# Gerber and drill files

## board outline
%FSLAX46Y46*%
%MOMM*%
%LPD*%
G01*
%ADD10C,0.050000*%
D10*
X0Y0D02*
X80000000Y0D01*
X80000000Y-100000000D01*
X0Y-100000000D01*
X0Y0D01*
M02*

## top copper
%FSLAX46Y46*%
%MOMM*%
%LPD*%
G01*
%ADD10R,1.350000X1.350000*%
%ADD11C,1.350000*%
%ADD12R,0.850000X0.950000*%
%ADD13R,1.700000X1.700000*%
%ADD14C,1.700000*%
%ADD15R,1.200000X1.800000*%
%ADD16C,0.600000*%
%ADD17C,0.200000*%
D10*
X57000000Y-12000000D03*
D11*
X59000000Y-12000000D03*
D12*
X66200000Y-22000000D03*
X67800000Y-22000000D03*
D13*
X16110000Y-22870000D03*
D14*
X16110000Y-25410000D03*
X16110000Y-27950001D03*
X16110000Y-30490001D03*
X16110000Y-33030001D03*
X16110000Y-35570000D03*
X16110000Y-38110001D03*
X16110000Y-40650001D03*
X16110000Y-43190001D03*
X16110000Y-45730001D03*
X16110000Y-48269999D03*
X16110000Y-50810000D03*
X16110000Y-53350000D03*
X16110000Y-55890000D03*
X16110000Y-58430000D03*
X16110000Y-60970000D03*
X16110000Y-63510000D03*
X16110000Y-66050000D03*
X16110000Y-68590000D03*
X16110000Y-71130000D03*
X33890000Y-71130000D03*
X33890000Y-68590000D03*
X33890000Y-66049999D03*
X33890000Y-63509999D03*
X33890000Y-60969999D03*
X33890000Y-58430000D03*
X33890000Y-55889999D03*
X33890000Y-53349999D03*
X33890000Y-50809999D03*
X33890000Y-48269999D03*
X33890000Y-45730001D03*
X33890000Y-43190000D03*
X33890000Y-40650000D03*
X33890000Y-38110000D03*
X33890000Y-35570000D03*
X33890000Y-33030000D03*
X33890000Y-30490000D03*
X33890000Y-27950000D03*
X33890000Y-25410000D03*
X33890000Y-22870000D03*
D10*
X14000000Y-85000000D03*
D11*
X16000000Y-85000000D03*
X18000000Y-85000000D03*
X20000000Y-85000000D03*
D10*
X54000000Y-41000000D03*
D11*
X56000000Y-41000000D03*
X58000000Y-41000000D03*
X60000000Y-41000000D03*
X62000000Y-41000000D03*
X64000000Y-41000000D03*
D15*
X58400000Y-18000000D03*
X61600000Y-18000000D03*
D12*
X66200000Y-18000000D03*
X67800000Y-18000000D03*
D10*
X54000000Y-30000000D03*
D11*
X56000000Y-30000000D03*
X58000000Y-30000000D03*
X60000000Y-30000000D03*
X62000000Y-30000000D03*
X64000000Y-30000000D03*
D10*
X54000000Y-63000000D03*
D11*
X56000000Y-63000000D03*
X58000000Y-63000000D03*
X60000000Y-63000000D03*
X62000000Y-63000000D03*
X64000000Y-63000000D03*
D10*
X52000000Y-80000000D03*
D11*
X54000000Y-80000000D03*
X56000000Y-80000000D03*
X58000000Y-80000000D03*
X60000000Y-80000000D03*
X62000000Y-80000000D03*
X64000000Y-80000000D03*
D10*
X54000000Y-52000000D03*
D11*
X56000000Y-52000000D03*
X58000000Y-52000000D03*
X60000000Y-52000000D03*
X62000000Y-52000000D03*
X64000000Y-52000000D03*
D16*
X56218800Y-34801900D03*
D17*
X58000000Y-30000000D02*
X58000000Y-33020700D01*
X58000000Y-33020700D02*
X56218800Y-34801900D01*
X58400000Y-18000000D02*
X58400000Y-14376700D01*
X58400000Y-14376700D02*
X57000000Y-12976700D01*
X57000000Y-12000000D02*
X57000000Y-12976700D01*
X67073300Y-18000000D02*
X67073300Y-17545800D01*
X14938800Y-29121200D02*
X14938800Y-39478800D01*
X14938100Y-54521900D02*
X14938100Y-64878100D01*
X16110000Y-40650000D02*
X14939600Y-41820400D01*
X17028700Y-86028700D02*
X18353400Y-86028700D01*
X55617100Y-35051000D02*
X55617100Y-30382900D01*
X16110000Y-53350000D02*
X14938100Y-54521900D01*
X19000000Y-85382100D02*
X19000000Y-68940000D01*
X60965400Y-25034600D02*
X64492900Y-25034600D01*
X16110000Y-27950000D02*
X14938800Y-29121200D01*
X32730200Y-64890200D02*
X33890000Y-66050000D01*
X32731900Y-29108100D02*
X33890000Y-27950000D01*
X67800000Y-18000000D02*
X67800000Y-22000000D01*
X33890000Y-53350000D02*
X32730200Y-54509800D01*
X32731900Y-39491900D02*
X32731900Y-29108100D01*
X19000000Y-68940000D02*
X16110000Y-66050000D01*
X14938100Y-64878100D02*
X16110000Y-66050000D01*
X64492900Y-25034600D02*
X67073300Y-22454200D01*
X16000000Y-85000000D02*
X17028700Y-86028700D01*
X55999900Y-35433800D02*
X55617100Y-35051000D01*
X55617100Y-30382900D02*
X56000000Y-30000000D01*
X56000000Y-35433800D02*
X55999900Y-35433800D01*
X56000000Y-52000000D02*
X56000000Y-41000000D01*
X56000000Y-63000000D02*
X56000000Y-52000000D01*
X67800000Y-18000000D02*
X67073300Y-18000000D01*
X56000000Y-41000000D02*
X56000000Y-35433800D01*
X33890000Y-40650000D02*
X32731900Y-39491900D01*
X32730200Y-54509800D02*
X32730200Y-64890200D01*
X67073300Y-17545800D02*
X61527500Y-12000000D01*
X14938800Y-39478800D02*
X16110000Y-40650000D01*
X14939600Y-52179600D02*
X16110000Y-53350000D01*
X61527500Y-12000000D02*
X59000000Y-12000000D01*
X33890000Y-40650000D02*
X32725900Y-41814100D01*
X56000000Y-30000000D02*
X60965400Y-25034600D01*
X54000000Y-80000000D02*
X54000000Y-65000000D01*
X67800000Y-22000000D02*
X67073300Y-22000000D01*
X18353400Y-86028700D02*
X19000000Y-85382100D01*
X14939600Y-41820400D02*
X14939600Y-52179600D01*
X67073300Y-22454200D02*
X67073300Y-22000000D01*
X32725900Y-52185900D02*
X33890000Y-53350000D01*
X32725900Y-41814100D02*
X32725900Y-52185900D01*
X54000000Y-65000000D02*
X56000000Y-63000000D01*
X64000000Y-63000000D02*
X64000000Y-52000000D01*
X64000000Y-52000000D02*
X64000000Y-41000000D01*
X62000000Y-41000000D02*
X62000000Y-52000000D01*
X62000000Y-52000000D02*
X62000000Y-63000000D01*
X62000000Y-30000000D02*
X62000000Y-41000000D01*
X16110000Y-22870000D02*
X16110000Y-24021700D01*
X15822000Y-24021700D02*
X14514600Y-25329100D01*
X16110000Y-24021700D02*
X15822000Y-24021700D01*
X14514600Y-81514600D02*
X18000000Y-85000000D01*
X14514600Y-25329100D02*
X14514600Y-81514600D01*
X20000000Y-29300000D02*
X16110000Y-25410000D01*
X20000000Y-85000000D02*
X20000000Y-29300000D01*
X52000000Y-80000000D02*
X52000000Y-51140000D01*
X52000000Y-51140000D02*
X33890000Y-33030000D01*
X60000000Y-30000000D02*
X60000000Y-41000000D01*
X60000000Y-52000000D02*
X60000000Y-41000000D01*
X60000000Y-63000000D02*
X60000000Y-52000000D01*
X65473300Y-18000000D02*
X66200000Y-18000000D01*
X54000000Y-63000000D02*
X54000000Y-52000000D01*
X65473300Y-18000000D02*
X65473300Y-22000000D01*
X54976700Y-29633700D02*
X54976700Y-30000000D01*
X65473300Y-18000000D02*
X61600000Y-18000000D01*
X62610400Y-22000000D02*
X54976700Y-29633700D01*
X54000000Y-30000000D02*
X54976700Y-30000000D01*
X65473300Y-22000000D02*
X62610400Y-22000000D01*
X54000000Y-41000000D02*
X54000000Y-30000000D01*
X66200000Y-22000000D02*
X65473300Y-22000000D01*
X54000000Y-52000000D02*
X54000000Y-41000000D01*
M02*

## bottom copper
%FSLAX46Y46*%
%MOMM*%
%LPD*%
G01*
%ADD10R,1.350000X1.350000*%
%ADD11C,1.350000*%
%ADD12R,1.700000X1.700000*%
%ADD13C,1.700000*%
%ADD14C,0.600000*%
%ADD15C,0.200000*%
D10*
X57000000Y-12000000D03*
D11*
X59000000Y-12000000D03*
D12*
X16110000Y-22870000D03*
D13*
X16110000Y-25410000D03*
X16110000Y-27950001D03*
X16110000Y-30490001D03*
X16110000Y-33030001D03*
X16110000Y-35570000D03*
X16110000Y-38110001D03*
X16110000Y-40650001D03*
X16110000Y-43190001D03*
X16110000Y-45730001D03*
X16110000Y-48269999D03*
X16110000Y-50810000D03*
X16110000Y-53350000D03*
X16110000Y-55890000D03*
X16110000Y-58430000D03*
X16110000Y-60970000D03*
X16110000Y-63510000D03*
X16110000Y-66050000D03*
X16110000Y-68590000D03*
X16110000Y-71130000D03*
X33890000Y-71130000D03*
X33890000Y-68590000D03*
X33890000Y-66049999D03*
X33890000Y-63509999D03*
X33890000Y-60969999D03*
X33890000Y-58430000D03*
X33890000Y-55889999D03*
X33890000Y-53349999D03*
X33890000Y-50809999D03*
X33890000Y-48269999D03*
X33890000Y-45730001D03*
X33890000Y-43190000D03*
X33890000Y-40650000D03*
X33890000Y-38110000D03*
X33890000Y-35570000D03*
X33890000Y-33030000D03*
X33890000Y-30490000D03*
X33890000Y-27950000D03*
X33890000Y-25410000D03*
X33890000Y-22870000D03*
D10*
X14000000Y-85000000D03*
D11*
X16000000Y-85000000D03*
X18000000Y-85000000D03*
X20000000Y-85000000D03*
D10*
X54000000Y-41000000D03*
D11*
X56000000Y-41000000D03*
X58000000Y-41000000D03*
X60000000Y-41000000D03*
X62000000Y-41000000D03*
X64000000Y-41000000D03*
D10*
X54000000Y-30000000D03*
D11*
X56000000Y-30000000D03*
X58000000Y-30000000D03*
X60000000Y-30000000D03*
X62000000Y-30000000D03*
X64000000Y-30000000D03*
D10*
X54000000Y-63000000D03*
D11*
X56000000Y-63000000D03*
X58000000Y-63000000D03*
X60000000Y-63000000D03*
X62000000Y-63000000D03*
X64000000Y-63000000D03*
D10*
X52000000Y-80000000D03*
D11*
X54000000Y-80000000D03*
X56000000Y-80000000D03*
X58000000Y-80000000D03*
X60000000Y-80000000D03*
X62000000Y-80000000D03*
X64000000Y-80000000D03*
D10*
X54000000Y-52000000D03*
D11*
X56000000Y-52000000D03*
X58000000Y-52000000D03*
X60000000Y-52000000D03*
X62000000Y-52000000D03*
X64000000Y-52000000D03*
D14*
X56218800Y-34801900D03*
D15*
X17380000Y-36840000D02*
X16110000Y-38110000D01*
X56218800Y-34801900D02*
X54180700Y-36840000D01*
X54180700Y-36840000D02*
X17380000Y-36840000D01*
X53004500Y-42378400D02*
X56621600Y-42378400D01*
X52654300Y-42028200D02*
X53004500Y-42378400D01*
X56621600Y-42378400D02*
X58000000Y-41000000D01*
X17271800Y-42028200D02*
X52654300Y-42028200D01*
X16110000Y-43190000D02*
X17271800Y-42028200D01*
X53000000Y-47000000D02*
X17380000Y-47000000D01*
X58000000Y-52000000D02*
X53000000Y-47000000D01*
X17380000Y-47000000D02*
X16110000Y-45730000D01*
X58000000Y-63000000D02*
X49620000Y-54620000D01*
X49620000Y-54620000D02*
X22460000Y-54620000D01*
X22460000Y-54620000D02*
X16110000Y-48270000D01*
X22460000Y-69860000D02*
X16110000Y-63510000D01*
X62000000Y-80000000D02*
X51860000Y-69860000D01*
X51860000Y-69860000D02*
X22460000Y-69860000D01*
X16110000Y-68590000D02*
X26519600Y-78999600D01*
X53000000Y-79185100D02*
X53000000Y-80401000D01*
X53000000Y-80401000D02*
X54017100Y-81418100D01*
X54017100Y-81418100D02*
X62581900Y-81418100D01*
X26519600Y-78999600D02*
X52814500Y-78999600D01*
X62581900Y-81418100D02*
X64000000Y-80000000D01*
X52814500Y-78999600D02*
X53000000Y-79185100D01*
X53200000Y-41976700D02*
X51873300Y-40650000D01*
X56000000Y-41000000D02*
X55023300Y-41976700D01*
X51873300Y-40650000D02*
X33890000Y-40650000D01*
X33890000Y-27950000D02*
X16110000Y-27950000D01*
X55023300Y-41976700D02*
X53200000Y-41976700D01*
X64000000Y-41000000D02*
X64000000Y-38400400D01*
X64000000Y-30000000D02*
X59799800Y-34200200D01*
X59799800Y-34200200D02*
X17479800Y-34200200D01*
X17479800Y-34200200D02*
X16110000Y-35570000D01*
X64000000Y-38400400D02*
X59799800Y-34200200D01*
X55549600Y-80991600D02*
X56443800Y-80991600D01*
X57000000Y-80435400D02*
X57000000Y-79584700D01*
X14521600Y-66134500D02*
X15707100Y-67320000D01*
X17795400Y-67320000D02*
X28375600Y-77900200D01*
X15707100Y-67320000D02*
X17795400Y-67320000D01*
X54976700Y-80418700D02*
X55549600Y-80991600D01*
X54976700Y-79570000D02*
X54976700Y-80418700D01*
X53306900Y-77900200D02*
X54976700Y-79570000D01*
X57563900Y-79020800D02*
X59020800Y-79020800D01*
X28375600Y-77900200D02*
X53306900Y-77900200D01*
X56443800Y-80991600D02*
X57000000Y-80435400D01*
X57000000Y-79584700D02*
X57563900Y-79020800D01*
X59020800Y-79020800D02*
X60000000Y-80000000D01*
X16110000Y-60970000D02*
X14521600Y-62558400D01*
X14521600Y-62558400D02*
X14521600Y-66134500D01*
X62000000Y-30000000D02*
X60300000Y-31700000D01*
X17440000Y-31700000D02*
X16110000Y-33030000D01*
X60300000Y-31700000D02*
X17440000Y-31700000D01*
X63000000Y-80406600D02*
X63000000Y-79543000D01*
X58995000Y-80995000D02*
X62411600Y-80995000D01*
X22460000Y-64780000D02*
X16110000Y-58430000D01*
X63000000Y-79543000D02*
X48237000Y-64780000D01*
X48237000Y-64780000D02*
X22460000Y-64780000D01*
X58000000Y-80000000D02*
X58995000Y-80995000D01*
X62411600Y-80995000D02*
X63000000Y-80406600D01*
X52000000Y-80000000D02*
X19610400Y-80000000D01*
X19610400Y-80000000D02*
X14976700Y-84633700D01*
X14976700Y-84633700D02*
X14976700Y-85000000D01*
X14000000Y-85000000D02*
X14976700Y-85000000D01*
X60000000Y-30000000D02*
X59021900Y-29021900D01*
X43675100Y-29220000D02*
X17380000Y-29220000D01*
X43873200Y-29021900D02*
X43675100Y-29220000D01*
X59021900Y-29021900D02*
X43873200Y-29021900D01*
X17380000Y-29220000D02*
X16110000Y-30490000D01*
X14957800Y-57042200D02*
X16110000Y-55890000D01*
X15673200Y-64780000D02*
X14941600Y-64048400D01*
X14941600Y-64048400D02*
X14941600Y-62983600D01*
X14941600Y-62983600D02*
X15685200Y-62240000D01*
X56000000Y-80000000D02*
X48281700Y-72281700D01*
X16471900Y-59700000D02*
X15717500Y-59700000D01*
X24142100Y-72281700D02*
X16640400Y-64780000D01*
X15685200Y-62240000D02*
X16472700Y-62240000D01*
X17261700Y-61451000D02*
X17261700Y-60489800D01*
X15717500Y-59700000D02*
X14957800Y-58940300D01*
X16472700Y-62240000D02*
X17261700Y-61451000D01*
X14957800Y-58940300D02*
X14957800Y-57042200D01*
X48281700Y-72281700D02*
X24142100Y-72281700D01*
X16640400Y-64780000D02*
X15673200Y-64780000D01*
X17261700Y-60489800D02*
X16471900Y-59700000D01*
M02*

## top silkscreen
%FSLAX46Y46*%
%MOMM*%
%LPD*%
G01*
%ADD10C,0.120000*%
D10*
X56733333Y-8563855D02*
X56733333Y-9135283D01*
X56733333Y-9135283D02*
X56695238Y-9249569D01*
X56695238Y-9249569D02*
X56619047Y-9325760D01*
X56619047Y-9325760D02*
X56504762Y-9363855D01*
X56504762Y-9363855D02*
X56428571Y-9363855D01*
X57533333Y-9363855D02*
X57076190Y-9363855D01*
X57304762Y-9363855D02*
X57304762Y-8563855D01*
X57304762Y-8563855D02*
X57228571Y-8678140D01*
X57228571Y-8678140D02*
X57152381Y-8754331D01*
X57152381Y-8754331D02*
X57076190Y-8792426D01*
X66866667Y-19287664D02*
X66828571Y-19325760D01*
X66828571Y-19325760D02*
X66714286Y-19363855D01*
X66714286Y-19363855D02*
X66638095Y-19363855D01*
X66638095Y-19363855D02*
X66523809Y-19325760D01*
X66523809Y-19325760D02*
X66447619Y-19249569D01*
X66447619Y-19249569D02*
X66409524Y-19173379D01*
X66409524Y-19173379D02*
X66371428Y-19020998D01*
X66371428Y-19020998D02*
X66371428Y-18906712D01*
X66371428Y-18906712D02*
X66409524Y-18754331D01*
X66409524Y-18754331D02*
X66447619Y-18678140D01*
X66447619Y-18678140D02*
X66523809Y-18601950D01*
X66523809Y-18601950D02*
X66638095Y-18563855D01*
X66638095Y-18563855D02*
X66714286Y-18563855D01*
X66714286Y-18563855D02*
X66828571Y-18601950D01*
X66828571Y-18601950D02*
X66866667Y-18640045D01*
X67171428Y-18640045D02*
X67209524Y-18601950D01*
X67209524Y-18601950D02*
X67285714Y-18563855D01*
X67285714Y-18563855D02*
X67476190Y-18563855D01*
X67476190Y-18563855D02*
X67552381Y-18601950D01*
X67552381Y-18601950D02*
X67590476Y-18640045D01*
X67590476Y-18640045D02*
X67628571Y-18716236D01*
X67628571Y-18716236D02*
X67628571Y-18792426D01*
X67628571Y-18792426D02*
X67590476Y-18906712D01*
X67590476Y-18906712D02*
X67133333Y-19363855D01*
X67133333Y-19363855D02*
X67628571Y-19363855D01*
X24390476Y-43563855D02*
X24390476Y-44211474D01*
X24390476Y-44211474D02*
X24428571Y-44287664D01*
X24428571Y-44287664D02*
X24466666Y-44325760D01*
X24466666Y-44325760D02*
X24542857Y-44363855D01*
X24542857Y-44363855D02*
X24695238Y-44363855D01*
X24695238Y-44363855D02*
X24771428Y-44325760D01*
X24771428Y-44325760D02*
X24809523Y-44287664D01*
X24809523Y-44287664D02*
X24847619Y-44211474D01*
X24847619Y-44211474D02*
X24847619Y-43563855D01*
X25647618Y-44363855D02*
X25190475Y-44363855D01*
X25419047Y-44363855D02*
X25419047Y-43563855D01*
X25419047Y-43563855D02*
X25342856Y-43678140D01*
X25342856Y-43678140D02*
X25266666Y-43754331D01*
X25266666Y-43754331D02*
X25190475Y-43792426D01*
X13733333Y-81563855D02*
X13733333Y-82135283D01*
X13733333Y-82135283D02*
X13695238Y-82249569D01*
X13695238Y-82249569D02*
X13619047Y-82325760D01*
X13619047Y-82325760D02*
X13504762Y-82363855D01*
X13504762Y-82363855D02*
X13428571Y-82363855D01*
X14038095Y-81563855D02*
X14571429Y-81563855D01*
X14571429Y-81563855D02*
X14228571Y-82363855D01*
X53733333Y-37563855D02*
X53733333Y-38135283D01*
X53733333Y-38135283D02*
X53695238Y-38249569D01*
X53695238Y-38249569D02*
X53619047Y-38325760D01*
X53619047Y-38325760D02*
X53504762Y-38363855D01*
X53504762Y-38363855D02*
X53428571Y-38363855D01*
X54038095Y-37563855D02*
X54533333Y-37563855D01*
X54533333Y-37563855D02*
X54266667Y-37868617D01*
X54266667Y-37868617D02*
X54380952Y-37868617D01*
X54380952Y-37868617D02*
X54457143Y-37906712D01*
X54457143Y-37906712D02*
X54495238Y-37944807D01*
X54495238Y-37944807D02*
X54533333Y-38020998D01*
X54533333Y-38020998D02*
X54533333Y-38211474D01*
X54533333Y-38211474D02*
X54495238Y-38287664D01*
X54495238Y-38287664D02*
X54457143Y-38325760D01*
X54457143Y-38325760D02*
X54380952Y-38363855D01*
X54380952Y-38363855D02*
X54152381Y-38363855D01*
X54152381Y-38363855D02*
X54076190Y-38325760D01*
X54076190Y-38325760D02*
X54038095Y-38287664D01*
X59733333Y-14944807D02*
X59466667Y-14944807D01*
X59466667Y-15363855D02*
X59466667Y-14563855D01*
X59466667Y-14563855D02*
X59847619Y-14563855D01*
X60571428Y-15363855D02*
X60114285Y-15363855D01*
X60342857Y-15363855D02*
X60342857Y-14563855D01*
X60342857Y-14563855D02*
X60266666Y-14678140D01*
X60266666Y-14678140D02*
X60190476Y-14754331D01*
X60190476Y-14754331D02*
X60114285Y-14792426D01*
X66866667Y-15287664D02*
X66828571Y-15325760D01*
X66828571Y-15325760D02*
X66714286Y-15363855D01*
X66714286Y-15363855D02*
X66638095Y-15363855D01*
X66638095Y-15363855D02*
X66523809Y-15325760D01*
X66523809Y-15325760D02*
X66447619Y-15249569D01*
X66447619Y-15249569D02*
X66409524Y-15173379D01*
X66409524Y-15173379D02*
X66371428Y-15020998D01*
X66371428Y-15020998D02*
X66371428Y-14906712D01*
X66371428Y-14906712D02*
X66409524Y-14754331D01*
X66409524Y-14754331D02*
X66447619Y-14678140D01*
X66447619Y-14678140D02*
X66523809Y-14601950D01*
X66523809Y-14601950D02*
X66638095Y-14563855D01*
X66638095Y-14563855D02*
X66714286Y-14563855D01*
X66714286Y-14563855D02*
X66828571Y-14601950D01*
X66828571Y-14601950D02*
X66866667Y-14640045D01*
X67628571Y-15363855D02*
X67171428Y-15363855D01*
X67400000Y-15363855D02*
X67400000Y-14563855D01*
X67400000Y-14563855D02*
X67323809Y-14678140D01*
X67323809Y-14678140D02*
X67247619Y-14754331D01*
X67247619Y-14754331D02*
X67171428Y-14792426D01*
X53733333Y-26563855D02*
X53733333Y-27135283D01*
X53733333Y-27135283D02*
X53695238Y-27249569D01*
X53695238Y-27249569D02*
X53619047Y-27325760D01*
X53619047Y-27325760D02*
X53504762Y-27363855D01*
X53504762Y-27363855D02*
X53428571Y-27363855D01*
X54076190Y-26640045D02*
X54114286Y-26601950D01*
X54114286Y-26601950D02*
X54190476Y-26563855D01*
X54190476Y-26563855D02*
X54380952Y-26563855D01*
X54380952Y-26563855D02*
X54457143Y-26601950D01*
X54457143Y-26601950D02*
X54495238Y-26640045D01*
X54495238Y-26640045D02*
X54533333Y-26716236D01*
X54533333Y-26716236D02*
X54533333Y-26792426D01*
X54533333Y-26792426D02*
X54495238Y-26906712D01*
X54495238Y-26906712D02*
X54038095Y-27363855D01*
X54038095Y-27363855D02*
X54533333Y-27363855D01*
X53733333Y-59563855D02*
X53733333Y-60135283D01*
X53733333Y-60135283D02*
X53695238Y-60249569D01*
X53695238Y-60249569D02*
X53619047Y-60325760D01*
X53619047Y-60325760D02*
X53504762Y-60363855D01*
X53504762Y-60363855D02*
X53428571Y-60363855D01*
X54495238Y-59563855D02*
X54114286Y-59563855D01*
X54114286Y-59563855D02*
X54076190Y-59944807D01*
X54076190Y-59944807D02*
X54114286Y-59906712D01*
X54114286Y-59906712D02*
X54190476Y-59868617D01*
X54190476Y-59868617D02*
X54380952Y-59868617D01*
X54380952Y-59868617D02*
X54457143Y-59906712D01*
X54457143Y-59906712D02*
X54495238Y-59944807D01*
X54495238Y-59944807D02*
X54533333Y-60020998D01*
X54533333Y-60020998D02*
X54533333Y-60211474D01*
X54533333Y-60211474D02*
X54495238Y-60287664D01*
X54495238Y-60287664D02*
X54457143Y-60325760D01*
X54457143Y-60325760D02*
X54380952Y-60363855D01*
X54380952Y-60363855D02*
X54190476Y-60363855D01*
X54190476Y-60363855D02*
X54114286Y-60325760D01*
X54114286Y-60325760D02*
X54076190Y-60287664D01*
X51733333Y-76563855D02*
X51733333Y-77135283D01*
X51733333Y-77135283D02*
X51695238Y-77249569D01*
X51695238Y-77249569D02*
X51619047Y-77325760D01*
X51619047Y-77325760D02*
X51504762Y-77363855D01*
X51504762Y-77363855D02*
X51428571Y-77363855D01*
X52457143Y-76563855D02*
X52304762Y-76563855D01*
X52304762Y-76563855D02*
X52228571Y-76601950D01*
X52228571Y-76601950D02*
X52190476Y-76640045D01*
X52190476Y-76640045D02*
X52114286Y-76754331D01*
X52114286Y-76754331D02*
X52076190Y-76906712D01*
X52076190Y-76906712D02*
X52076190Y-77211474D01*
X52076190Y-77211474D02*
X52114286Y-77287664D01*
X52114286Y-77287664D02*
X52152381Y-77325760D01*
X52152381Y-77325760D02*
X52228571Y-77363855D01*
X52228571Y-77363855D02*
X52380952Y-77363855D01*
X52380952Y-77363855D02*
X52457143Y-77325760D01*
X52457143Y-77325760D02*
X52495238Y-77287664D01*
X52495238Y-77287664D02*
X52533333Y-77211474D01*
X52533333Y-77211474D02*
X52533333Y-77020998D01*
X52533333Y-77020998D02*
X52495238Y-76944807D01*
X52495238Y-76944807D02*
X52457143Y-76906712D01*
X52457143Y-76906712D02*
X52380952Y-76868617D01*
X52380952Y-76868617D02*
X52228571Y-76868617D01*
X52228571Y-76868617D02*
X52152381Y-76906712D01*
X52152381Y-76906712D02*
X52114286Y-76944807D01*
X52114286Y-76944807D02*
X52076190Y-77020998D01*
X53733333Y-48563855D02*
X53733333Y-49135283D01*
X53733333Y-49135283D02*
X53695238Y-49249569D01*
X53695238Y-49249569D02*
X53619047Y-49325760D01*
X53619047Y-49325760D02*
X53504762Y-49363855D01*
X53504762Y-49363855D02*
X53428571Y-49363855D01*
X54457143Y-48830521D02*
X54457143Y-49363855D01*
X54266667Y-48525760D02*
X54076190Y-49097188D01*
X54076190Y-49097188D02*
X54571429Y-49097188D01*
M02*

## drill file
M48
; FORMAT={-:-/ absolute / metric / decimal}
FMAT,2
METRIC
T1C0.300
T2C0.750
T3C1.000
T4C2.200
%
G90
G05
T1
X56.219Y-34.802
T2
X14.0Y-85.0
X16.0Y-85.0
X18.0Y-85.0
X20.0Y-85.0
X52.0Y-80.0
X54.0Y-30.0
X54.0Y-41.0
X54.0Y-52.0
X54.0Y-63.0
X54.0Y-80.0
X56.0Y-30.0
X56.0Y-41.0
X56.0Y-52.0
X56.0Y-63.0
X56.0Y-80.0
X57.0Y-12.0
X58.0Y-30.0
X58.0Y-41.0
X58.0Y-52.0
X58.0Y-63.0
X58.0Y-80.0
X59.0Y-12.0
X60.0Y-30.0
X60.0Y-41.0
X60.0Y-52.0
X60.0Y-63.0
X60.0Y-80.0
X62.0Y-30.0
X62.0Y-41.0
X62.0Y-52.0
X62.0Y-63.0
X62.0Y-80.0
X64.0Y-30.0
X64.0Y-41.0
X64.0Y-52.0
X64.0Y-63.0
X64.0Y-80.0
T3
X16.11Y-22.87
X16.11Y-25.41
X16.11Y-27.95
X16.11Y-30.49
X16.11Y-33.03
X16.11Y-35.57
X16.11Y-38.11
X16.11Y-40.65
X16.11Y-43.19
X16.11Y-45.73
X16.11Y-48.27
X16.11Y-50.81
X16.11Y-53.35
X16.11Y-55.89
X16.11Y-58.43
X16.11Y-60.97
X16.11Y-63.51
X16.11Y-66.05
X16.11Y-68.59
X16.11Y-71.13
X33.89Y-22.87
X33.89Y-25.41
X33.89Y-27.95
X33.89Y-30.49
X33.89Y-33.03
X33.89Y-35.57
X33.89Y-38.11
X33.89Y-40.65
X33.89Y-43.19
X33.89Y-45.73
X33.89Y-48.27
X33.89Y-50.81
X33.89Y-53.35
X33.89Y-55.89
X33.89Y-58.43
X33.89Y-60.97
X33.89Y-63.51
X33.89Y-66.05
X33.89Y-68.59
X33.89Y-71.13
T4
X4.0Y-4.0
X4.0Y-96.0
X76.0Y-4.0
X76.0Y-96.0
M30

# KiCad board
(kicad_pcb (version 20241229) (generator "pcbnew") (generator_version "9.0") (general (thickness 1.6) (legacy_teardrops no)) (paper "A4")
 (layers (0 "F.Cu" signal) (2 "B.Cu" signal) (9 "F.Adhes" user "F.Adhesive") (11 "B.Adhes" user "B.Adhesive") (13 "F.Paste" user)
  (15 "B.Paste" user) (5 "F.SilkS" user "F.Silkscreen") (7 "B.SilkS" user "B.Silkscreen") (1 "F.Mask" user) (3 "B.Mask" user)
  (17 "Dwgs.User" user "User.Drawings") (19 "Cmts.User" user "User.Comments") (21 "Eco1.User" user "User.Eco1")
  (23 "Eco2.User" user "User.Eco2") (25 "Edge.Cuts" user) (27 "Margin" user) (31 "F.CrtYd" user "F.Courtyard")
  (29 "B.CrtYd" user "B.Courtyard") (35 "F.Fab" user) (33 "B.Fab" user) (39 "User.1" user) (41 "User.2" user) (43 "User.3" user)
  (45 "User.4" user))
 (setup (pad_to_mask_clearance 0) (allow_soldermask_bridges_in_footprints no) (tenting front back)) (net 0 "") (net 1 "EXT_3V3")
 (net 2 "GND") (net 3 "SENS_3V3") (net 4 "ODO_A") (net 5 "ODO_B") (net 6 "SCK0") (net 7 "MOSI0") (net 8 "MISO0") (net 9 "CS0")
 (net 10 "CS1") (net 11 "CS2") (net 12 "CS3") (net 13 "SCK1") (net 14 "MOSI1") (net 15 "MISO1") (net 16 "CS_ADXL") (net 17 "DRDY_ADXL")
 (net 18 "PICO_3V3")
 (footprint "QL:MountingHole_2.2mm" (layer "F.Cu") (at 76 4)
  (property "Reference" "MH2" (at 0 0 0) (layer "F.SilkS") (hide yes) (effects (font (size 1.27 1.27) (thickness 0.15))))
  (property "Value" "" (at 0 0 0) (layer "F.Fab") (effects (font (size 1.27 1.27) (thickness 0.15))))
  (pad "" np_thru_hole circle (at 0 0) (size 2.2 2.2) (drill 2.2) (layers "*.Cu" "*.Mask")))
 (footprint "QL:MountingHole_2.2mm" (layer "F.Cu") (at 76 96)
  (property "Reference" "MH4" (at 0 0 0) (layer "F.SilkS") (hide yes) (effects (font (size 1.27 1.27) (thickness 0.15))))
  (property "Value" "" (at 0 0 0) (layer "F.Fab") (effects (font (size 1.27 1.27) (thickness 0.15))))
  (pad "" np_thru_hole circle (at 0 0) (size 2.2 2.2) (drill 2.2) (layers "*.Cu" "*.Mask")))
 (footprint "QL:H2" (layer "F.Cu") (at 57 12)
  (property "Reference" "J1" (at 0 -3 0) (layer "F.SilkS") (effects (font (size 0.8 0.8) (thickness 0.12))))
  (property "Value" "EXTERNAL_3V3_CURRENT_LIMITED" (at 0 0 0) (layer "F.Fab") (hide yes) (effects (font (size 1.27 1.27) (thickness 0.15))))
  (pad "1" thru_hole rect (at 0 0) (size 1.35 1.35) (drill 0.75) (layers "*.Cu" "*.Mask") (remove_unused_layers no) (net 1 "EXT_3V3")
   (thermal_bridge_angle 45))
  (pad "2" thru_hole circle (at 2 0) (size 1.35 1.35) (drill 0.75) (layers "*.Cu" "*.Mask") (remove_unused_layers no) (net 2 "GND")))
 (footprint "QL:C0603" (layer "F.Cu") (at 67 22)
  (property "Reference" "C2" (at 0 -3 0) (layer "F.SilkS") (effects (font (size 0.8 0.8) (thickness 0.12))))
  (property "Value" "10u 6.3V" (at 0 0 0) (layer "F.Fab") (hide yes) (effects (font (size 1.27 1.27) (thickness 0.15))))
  (pad "1" smd rect (at -0.8 0) (size 0.85 0.95) (layers "F.Cu" "F.Mask" "F.Paste") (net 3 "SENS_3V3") (thermal_bridge_angle 45))
  (pad "2" smd rect (at 0.8 0) (size 0.85 0.95) (layers "F.Cu" "F.Mask" "F.Paste") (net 2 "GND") (thermal_bridge_angle 45)))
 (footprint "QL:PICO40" (layer "F.Cu") (at 25 47)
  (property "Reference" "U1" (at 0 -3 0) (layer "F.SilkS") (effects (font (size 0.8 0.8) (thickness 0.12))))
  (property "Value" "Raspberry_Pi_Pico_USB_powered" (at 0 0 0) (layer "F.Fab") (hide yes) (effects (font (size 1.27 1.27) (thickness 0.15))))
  (pad "1" thru_hole rect (at -8.89 -24.13) (size 1.7 1.7) (drill 1) (layers "*.Cu" "*.Mask") (remove_unused_layers no) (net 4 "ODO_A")
   (thermal_bridge_angle 45))
  (pad "2" thru_hole circle (at -8.89 -21.59) (size 1.7 1.7) (drill 1) (layers "*.Cu" "*.Mask") (remove_unused_layers no) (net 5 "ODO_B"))
  (pad "3" thru_hole circle (at -8.89 -19.049999) (size 1.7 1.7) (drill 1) (layers "*.Cu" "*.Mask") (remove_unused_layers no) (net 2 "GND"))
  (pad "4" thru_hole circle (at -8.89 -16.509999) (size 1.7 1.7) (drill 1) (layers "*.Cu" "*.Mask") (remove_unused_layers no) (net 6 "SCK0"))
  (pad "5" thru_hole circle (at -8.89 -13.969999) (size 1.7 1.7) (drill 1) (layers "*.Cu" "*.Mask") (remove_unused_layers no)
   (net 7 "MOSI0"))
  (pad "6" thru_hole circle (at -8.89 -11.43) (size 1.7 1.7) (drill 1) (layers "*.Cu" "*.Mask") (remove_unused_layers no) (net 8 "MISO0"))
  (pad "7" thru_hole circle (at -8.89 -8.889999) (size 1.7 1.7) (drill 1) (layers "*.Cu" "*.Mask") (remove_unused_layers no) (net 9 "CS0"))
  (pad "8" thru_hole circle (at -8.89 -6.349999) (size 1.7 1.7) (drill 1) (layers "*.Cu" "*.Mask") (remove_unused_layers no) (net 2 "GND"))
  (pad "9" thru_hole circle (at -8.89 -3.809999) (size 1.7 1.7) (drill 1) (layers "*.Cu" "*.Mask") (remove_unused_layers no) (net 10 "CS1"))
  (pad "10" thru_hole circle (at -8.89 -1.269999) (size 1.7 1.7) (drill 1) (layers "*.Cu" "*.Mask") (remove_unused_layers no) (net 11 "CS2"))
  (pad "11" thru_hole circle (at -8.89 1.269999) (size 1.7 1.7) (drill 1) (layers "*.Cu" "*.Mask") (remove_unused_layers no) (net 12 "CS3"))
  (pad "12" thru_hole circle (at -8.89 3.81) (size 1.7 1.7) (drill 1) (layers "*.Cu" "*.Mask") (remove_unused_layers no))
  (pad "13" thru_hole circle (at -8.89 6.35) (size 1.7 1.7) (drill 1) (layers "*.Cu" "*.Mask") (remove_unused_layers no) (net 2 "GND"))
  (pad "14" thru_hole circle (at -8.89 8.89) (size 1.7 1.7) (drill 1) (layers "*.Cu" "*.Mask") (remove_unused_layers no) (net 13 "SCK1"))
  (pad "15" thru_hole circle (at -8.89 11.43) (size 1.7 1.7) (drill 1) (layers "*.Cu" "*.Mask") (remove_unused_layers no) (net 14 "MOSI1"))
  (pad "16" thru_hole circle (at -8.89 13.97) (size 1.7 1.7) (drill 1) (layers "*.Cu" "*.Mask") (remove_unused_layers no) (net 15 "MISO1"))
  (pad "17" thru_hole circle (at -8.89 16.51) (size 1.7 1.7) (drill 1) (layers "*.Cu" "*.Mask") (remove_unused_layers no) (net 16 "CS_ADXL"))
  (pad "18" thru_hole circle (at -8.89 19.05) (size 1.7 1.7) (drill 1) (layers "*.Cu" "*.Mask") (remove_unused_layers no) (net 2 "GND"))
  (pad "19" thru_hole circle (at -8.89 21.59) (size 1.7 1.7) (drill 1) (layers "*.Cu" "*.Mask") (remove_unused_layers no)
   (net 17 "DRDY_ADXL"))
  (pad "20" thru_hole circle (at -8.89 24.13) (size 1.7 1.7) (drill 1) (layers "*.Cu" "*.Mask") (remove_unused_layers no))
  (pad "21" thru_hole circle (at 8.89 24.13) (size 1.7 1.7) (drill 1) (layers "*.Cu" "*.Mask") (remove_unused_layers no))
  (pad "22" thru_hole circle (at 8.89 21.59) (size 1.7 1.7) (drill 1) (layers "*.Cu" "*.Mask") (remove_unused_layers no))
  (pad "23" thru_hole circle (at 8.89 19.049999) (size 1.7 1.7) (drill 1) (layers "*.Cu" "*.Mask") (remove_unused_layers no) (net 2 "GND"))
  (pad "24" thru_hole circle (at 8.89 16.509999) (size 1.7 1.7) (drill 1) (layers "*.Cu" "*.Mask") (remove_unused_layers no))
  (pad "25" thru_hole circle (at 8.89 13.969999) (size 1.7 1.7) (drill 1) (layers "*.Cu" "*.Mask") (remove_unused_layers no))
  (pad "26" thru_hole circle (at 8.89 11.43) (size 1.7 1.7) (drill 1) (layers "*.Cu" "*.Mask") (remove_unused_layers no))
  (pad "27" thru_hole circle (at 8.89 8.889999) (size 1.7 1.7) (drill 1) (layers "*.Cu" "*.Mask") (remove_unused_layers no))
  (pad "28" thru_hole circle (at 8.89 6.349999) (size 1.7 1.7) (drill 1) (layers "*.Cu" "*.Mask") (remove_unused_layers no) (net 2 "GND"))
  (pad "29" thru_hole circle (at 8.89 3.809999) (size 1.7 1.7) (drill 1) (layers "*.Cu" "*.Mask") (remove_unused_layers no))
  (pad "30" thru_hole circle (at 8.89 1.269999) (size 1.7 1.7) (drill 1) (layers "*.Cu" "*.Mask") (remove_unused_layers no))
  (pad "31" thru_hole circle (at 8.89 -1.269999) (size 1.7 1.7) (drill 1) (layers "*.Cu" "*.Mask") (remove_unused_layers no))
  (pad "32" thru_hole circle (at 8.89 -3.81) (size 1.7 1.7) (drill 1) (layers "*.Cu" "*.Mask") (remove_unused_layers no))
  (pad "33" thru_hole circle (at 8.89 -6.35) (size 1.7 1.7) (drill 1) (layers "*.Cu" "*.Mask") (remove_unused_layers no) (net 2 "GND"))
  (pad "34" thru_hole circle (at 8.89 -8.89) (size 1.7 1.7) (drill 1) (layers "*.Cu" "*.Mask") (remove_unused_layers no))
  (pad "35" thru_hole circle (at 8.89 -11.43) (size 1.7 1.7) (drill 1) (layers "*.Cu" "*.Mask") (remove_unused_layers no))
  (pad "36" thru_hole circle (at 8.89 -13.97) (size 1.7 1.7) (drill 1) (layers "*.Cu" "*.Mask") (remove_unused_layers no)
   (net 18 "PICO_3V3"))
  (pad "37" thru_hole circle (at 8.89 -16.51) (size 1.7 1.7) (drill 1) (layers "*.Cu" "*.Mask") (remove_unused_layers no))
  (pad "38" thru_hole circle (at 8.89 -19.05) (size 1.7 1.7) (drill 1) (layers "*.Cu" "*.Mask") (remove_unused_layers no) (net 2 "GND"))
  (pad "39" thru_hole circle (at 8.89 -21.59) (size 1.7 1.7) (drill 1) (layers "*.Cu" "*.Mask") (remove_unused_layers no))
  (pad "40" thru_hole circle (at 8.89 -24.13) (size 1.7 1.7) (drill 1) (layers "*.Cu" "*.Mask") (remove_unused_layers no)))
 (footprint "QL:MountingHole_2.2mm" (layer "F.Cu") (at 4 4)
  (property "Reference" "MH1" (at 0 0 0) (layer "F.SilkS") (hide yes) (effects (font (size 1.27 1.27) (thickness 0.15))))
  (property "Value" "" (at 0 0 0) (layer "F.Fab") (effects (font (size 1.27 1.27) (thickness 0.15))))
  (pad "" np_thru_hole circle (at 0 0) (size 2.2 2.2) (drill 2.2) (layers "*.Cu" "*.Mask")))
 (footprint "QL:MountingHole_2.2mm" (layer "F.Cu") (at 4 96)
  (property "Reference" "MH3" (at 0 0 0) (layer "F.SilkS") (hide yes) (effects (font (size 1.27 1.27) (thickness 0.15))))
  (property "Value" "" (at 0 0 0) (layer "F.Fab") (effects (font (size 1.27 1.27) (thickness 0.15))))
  (pad "" np_thru_hole circle (at 0 0) (size 2.2 2.2) (drill 2.2) (layers "*.Cu" "*.Mask")))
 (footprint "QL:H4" (layer "F.Cu") (at 14 85)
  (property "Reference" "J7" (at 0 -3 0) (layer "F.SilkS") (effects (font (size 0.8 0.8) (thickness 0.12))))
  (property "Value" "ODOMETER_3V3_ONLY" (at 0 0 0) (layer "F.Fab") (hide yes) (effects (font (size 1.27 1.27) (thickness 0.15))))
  (pad "1" thru_hole rect (at 0 0) (size 1.35 1.35) (drill 0.75) (layers "*.Cu" "*.Mask") (remove_unused_layers no) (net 18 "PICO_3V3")
   (thermal_bridge_angle 45))
  (pad "2" thru_hole circle (at 2 0) (size 1.35 1.35) (drill 0.75) (layers "*.Cu" "*.Mask") (remove_unused_layers no) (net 2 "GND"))
  (pad "3" thru_hole circle (at 4 0) (size 1.35 1.35) (drill 0.75) (layers "*.Cu" "*.Mask") (remove_unused_layers no) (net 4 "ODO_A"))
  (pad "4" thru_hole circle (at 6 0) (size 1.35 1.35) (drill 0.75) (layers "*.Cu" "*.Mask") (remove_unused_layers no) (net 5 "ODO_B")))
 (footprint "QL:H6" (layer "F.Cu") (at 54 41)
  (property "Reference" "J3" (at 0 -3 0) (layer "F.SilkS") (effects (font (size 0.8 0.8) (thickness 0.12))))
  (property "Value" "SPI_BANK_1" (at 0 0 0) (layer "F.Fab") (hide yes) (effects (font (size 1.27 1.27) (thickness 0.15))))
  (pad "1" thru_hole rect (at 0 0) (size 1.35 1.35) (drill 0.75) (layers "*.Cu" "*.Mask") (remove_unused_layers no) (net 3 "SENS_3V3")
   (thermal_bridge_angle 45))
  (pad "2" thru_hole circle (at 2 0) (size 1.35 1.35) (drill 0.75) (layers "*.Cu" "*.Mask") (remove_unused_layers no) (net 2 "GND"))
  (pad "3" thru_hole circle (at 4 0) (size 1.35 1.35) (drill 0.75) (layers "*.Cu" "*.Mask") (remove_unused_layers no) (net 10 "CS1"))
  (pad "4" thru_hole circle (at 6 0) (size 1.35 1.35) (drill 0.75) (layers "*.Cu" "*.Mask") (remove_unused_layers no) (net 6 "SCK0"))
  (pad "5" thru_hole circle (at 8 0) (size 1.35 1.35) (drill 0.75) (layers "*.Cu" "*.Mask") (remove_unused_layers no) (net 7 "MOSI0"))
  (pad "6" thru_hole circle (at 10 0) (size 1.35 1.35) (drill 0.75) (layers "*.Cu" "*.Mask") (remove_unused_layers no) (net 8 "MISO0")))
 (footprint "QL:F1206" (layer "F.Cu") (at 60 18)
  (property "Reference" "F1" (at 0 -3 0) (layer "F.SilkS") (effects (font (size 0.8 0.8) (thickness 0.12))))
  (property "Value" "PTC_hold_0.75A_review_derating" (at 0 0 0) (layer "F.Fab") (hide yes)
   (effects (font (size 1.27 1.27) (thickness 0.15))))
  (pad "1" smd rect (at -1.6 0) (size 1.2 1.8) (layers "F.Cu" "F.Mask" "F.Paste") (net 1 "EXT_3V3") (thermal_bridge_angle 45))
  (pad "2" smd rect (at 1.6 0) (size 1.2 1.8) (layers "F.Cu" "F.Mask" "F.Paste") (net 3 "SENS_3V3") (thermal_bridge_angle 45)))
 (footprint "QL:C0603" (layer "F.Cu") (at 67 18)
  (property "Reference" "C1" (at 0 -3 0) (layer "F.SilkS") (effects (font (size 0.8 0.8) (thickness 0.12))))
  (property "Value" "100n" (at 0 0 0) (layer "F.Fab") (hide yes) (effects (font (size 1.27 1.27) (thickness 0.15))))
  (pad "1" smd rect (at -0.8 0) (size 0.85 0.95) (layers "F.Cu" "F.Mask" "F.Paste") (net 3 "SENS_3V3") (thermal_bridge_angle 45))
  (pad "2" smd rect (at 0.8 0) (size 0.85 0.95) (layers "F.Cu" "F.Mask" "F.Paste") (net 2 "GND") (thermal_bridge_angle 45)))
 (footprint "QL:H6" (layer "F.Cu") (at 54 30)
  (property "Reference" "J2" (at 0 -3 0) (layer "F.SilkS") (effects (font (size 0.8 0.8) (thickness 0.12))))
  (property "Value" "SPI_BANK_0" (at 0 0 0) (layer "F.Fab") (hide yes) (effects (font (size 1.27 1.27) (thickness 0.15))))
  (pad "1" thru_hole rect (at 0 0) (size 1.35 1.35) (drill 0.75) (layers "*.Cu" "*.Mask") (remove_unused_layers no) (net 3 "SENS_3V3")
   (thermal_bridge_angle 45))
  (pad "2" thru_hole circle (at 2 0) (size 1.35 1.35) (drill 0.75) (layers "*.Cu" "*.Mask") (remove_unused_layers no) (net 2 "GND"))
  (pad "3" thru_hole circle (at 4 0) (size 1.35 1.35) (drill 0.75) (layers "*.Cu" "*.Mask") (remove_unused_layers no) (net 9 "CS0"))
  (pad "4" thru_hole circle (at 6 0) (size 1.35 1.35) (drill 0.75) (layers "*.Cu" "*.Mask") (remove_unused_layers no) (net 6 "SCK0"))
  (pad "5" thru_hole circle (at 8 0) (size 1.35 1.35) (drill 0.75) (layers "*.Cu" "*.Mask") (remove_unused_layers no) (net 7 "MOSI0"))
  (pad "6" thru_hole circle (at 10 0) (size 1.35 1.35) (drill 0.75) (layers "*.Cu" "*.Mask") (remove_unused_layers no) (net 8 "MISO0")))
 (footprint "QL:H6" (layer "F.Cu") (at 54 63)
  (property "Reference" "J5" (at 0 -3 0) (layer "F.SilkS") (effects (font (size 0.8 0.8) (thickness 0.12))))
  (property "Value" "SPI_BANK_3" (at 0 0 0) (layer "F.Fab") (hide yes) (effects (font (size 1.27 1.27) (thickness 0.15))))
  (pad "1" thru_hole rect (at 0 0) (size 1.35 1.35) (drill 0.75) (layers "*.Cu" "*.Mask") (remove_unused_layers no) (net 3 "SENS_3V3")
   (thermal_bridge_angle 45))
  (pad "2" thru_hole circle (at 2 0) (size 1.35 1.35) (drill 0.75) (layers "*.Cu" "*.Mask") (remove_unused_layers no) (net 2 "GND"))
  (pad "3" thru_hole circle (at 4 0) (size 1.35 1.35) (drill 0.75) (layers "*.Cu" "*.Mask") (remove_unused_layers no) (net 12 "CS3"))
  (pad "4" thru_hole circle (at 6 0) (size 1.35 1.35) (drill 0.75) (layers "*.Cu" "*.Mask") (remove_unused_layers no) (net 6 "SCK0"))
  (pad "5" thru_hole circle (at 8 0) (size 1.35 1.35) (drill 0.75) (layers "*.Cu" "*.Mask") (remove_unused_layers no) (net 7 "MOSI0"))
  (pad "6" thru_hole circle (at 10 0) (size 1.35 1.35) (drill 0.75) (layers "*.Cu" "*.Mask") (remove_unused_layers no) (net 8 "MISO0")))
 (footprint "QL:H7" (layer "F.Cu") (at 52 80)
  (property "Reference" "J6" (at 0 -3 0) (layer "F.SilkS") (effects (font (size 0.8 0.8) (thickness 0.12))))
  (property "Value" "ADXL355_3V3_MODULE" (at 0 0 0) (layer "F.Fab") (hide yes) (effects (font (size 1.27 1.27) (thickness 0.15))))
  (pad "1" thru_hole rect (at 0 0) (size 1.35 1.35) (drill 0.75) (layers "*.Cu" "*.Mask") (remove_unused_layers no) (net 18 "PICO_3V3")
   (thermal_bridge_angle 45))
  (pad "2" thru_hole circle (at 2 0) (size 1.35 1.35) (drill 0.75) (layers "*.Cu" "*.Mask") (remove_unused_layers no) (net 2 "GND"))
  (pad "3" thru_hole circle (at 4 0) (size 1.35 1.35) (drill 0.75) (layers "*.Cu" "*.Mask") (remove_unused_layers no) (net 13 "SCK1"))
  (pad "4" thru_hole circle (at 6 0) (size 1.35 1.35) (drill 0.75) (layers "*.Cu" "*.Mask") (remove_unused_layers no) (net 14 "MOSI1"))
  (pad "5" thru_hole circle (at 8 0) (size 1.35 1.35) (drill 0.75) (layers "*.Cu" "*.Mask") (remove_unused_layers no) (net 15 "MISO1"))
  (pad "6" thru_hole circle (at 10 0) (size 1.35 1.35) (drill 0.75) (layers "*.Cu" "*.Mask") (remove_unused_layers no) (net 16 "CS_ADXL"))
  (pad "7" thru_hole circle (at 12 0) (size 1.35 1.35) (drill 0.75) (layers "*.Cu" "*.Mask") (remove_unused_layers no) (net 17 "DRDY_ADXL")))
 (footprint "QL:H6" (layer "F.Cu") (at 54 52)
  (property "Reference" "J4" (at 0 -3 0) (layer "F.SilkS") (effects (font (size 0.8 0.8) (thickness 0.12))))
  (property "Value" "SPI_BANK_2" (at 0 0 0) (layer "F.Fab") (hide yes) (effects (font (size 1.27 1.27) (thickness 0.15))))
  (pad "1" thru_hole rect (at 0 0) (size 1.35 1.35) (drill 0.75) (layers "*.Cu" "*.Mask") (remove_unused_layers no) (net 3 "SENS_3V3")
   (thermal_bridge_angle 45))
  (pad "2" thru_hole circle (at 2 0) (size 1.35 1.35) (drill 0.75) (layers "*.Cu" "*.Mask") (remove_unused_layers no) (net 2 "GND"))
  (pad "3" thru_hole circle (at 4 0) (size 1.35 1.35) (drill 0.75) (layers "*.Cu" "*.Mask") (remove_unused_layers no) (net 11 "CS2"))
  (pad "4" thru_hole circle (at 6 0) (size 1.35 1.35) (drill 0.75) (layers "*.Cu" "*.Mask") (remove_unused_layers no) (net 6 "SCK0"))
  (pad "5" thru_hole circle (at 8 0) (size 1.35 1.35) (drill 0.75) (layers "*.Cu" "*.Mask") (remove_unused_layers no) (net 7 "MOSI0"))
  (pad "6" thru_hole circle (at 10 0) (size 1.35 1.35) (drill 0.75) (layers "*.Cu" "*.Mask") (remove_unused_layers no) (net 8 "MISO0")))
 (gr_rect (start 0 0) (end 80 100) (stroke (width 0.05) (type default)) (fill no) (layer "Edge.Cuts"))
 (segment (start 58 30) (end 58 33.0207) (width 0.2) (layer "F.Cu") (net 9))
 (segment (start 58 33.0207) (end 56.2188 34.8019) (width 0.2) (layer "F.Cu") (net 9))
 (via (at 56.2188 34.8019) (size 0.6) (drill 0.3) (layers "F.Cu" "B.Cu") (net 9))
 (segment (start 17.38 36.84) (end 16.11 38.11) (width 0.2) (layer "B.Cu") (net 9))
 (segment (start 56.2188 34.8019) (end 54.1807 36.84) (width 0.2) (layer "B.Cu") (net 9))
 (segment (start 54.1807 36.84) (end 17.38 36.84) (width 0.2) (layer "B.Cu") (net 9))
 (segment (start 53.0045 42.3784) (end 56.6216 42.3784) (width 0.2) (layer "B.Cu") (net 10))
 (segment (start 52.6543 42.0282) (end 53.0045 42.3784) (width 0.2) (layer "B.Cu") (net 10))
 (segment (start 56.6216 42.3784) (end 58 41) (width 0.2) (layer "B.Cu") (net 10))
 (segment (start 17.2718 42.0282) (end 52.6543 42.0282) (width 0.2) (layer "B.Cu") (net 10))
 (segment (start 16.11 43.19) (end 17.2718 42.0282) (width 0.2) (layer "B.Cu") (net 10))
 (segment (start 53 47) (end 17.38 47) (width 0.2) (layer "B.Cu") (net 11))
 (segment (start 58 52) (end 53 47) (width 0.2) (layer "B.Cu") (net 11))
 (segment (start 17.38 47) (end 16.11 45.73) (width 0.2) (layer "B.Cu") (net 11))
 (segment (start 58 63) (end 49.62 54.62) (width 0.2) (layer "B.Cu") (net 12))
 (segment (start 49.62 54.62) (end 22.46 54.62) (width 0.2) (layer "B.Cu") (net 12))
 (segment (start 22.46 54.62) (end 16.11 48.27) (width 0.2) (layer "B.Cu") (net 12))
 (segment (start 22.46 69.86) (end 16.11 63.51) (width 0.2) (layer "B.Cu") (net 16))
 (segment (start 62 80) (end 51.86 69.86) (width 0.2) (layer "B.Cu") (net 16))
 (segment (start 51.86 69.86) (end 22.46 69.86) (width 0.2) (layer "B.Cu") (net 16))
 (segment (start 16.11 68.59) (end 26.5196 78.9996) (width 0.2) (layer "B.Cu") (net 17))
 (segment (start 53 79.1851) (end 53 80.401) (width 0.2) (layer "B.Cu") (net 17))
 (segment (start 53 80.401) (end 54.0171 81.4181) (width 0.2) (layer "B.Cu") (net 17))
 (segment (start 54.0171 81.4181) (end 62.5819 81.4181) (width 0.2) (layer "B.Cu") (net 17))
 (segment (start 26.5196 78.9996) (end 52.8145 78.9996) (width 0.2) (layer "B.Cu") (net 17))
 (segment (start 62.5819 81.4181) (end 64 80) (width 0.2) (layer "B.Cu") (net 17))
 (segment (start 52.8145 78.9996) (end 53 79.1851) (width 0.2) (layer "B.Cu") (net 17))
 (segment (start 58.4 18) (end 58.4 14.3767) (width 0.2) (layer "F.Cu") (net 1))
 (segment (start 58.4 14.3767) (end 57 12.9767) (width 0.2) (layer "F.Cu") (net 1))
 (segment (start 57 12) (end 57 12.9767) (width 0.2) (layer "F.Cu") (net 1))
 (segment (start 67.0733 18) (end 67.0733 17.5458) (width 0.2) (layer "F.Cu") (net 2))
 (segment (start 14.9388 29.1212) (end 14.9388 39.4788) (width 0.2) (layer "F.Cu") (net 2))
 (segment (start 14.9381 54.5219) (end 14.9381 64.8781) (width 0.2) (layer "F.Cu") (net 2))
 (segment (start 16.11 40.65) (end 14.9396 41.8204) (width 0.2) (layer "F.Cu") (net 2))
 (segment (start 17.0287 86.0287) (end 18.3534 86.0287) (width 0.2) (layer "F.Cu") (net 2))
 (segment (start 55.6171 35.051) (end 55.6171 30.3829) (width 0.2) (layer "F.Cu") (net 2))
 (segment (start 16.11 53.35) (end 14.9381 54.5219) (width 0.2) (layer "F.Cu") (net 2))
 (segment (start 19 85.3821) (end 19 68.94) (width 0.2) (layer "F.Cu") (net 2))
 (segment (start 60.9654 25.0346) (end 64.4929 25.0346) (width 0.2) (layer "F.Cu") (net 2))
 (segment (start 16.11 27.95) (end 14.9388 29.1212) (width 0.2) (layer "F.Cu") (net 2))
 (segment (start 32.7302 64.8902) (end 33.89 66.05) (width 0.2) (layer "F.Cu") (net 2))
 (segment (start 32.7319 29.1081) (end 33.89 27.95) (width 0.2) (layer "F.Cu") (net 2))
 (segment (start 67.8 18) (end 67.8 22) (width 0.2) (layer "F.Cu") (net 2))
 (segment (start 33.89 53.35) (end 32.7302 54.5098) (width 0.2) (layer "F.Cu") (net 2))
 (segment (start 32.7319 39.4919) (end 32.7319 29.1081) (width 0.2) (layer "F.Cu") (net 2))
 (segment (start 19 68.94) (end 16.11 66.05) (width 0.2) (layer "F.Cu") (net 2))
 (segment (start 14.9381 64.8781) (end 16.11 66.05) (width 0.2) (layer "F.Cu") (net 2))
 (segment (start 64.4929 25.0346) (end 67.0733 22.4542) (width 0.2) (layer "F.Cu") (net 2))
 (segment (start 16 85) (end 17.0287 86.0287) (width 0.2) (layer "F.Cu") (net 2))
 (segment (start 55.9999 35.4338) (end 55.6171 35.051) (width 0.2) (layer "F.Cu") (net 2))
 (segment (start 55.6171 30.3829) (end 56 30) (width 0.2) (layer "F.Cu") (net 2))
 (segment (start 56 35.4338) (end 55.9999 35.4338) (width 0.2) (layer "F.Cu") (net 2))
 (segment (start 56 52) (end 56 41) (width 0.2) (layer "F.Cu") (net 2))
 (segment (start 56 63) (end 56 52) (width 0.2) (layer "F.Cu") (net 2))
 (segment (start 67.8 18) (end 67.0733 18) (width 0.2) (layer "F.Cu") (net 2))
 (segment (start 56 41) (end 56 35.4338) (width 0.2) (layer "F.Cu") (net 2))
 (segment (start 33.89 40.65) (end 32.7319 39.4919) (width 0.2) (layer "F.Cu") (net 2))
 (segment (start 32.7302 54.5098) (end 32.7302 64.8902) (width 0.2) (layer "F.Cu") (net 2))
 (segment (start 67.0733 17.5458) (end 61.5275 12) (width 0.2) (layer "F.Cu") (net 2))
 (segment (start 14.9388 39.4788) (end 16.11 40.65) (width 0.2) (layer "F.Cu") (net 2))
 (segment (start 14.9396 52.1796) (end 16.11 53.35) (width 0.2) (layer "F.Cu") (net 2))
 (segment (start 61.5275 12) (end 59 12) (width 0.2) (layer "F.Cu") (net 2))
 (segment (start 33.89 40.65) (end 32.7259 41.8141) (width 0.2) (layer "F.Cu") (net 2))
 (segment (start 56 30) (end 60.9654 25.0346) (width 0.2) (layer "F.Cu") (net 2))
 (segment (start 54 80) (end 54 65) (width 0.2) (layer "F.Cu") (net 2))
 (segment (start 67.8 22) (end 67.0733 22) (width 0.2) (layer "F.Cu") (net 2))
 (segment (start 18.3534 86.0287) (end 19 85.3821) (width 0.2) (layer "F.Cu") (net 2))
 (segment (start 14.9396 41.8204) (end 14.9396 52.1796) (width 0.2) (layer "F.Cu") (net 2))
 (segment (start 67.0733 22.4542) (end 67.0733 22) (width 0.2) (layer "F.Cu") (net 2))
 (segment (start 32.7259 52.1859) (end 33.89 53.35) (width 0.2) (layer "F.Cu") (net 2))
 (segment (start 32.7259 41.8141) (end 32.7259 52.1859) (width 0.2) (layer "F.Cu") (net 2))
 (segment (start 54 65) (end 56 63) (width 0.2) (layer "F.Cu") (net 2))
 (segment (start 53.2 41.9767) (end 51.8733 40.65) (width 0.2) (layer "B.Cu") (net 2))
 (segment (start 56 41) (end 55.0233 41.9767) (width 0.2) (layer "B.Cu") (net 2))
 (segment (start 51.8733 40.65) (end 33.89 40.65) (width 0.2) (layer "B.Cu") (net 2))
 (segment (start 33.89 27.95) (end 16.11 27.95) (width 0.2) (layer "B.Cu") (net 2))
 (segment (start 55.0233 41.9767) (end 53.2 41.9767) (width 0.2) (layer "B.Cu") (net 2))
 (segment (start 64 63) (end 64 52) (width 0.2) (layer "F.Cu") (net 8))
 (segment (start 64 52) (end 64 41) (width 0.2) (layer "F.Cu") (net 8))
 (segment (start 64 41) (end 64 38.4004) (width 0.2) (layer "B.Cu") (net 8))
 (segment (start 64 30) (end 59.7998 34.2002) (width 0.2) (layer "B.Cu") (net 8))
 (segment (start 59.7998 34.2002) (end 17.4798 34.2002) (width 0.2) (layer "B.Cu") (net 8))
 (segment (start 17.4798 34.2002) (end 16.11 35.57) (width 0.2) (layer "B.Cu") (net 8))
 (segment (start 64 38.4004) (end 59.7998 34.2002) (width 0.2) (layer "B.Cu") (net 8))
 (segment (start 55.5496 80.9916) (end 56.4438 80.9916) (width 0.2) (layer "B.Cu") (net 15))
 (segment (start 57 80.4354) (end 57 79.5847) (width 0.2) (layer "B.Cu") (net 15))
 (segment (start 14.5216 66.1345) (end 15.7071 67.32) (width 0.2) (layer "B.Cu") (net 15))
 (segment (start 17.7954 67.32) (end 28.3756 77.9002) (width 0.2) (layer "B.Cu") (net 15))
 (segment (start 15.7071 67.32) (end 17.7954 67.32) (width 0.2) (layer "B.Cu") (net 15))
 (segment (start 54.9767 80.4187) (end 55.5496 80.9916) (width 0.2) (layer "B.Cu") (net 15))
 (segment (start 54.9767 79.57) (end 54.9767 80.4187) (width 0.2) (layer "B.Cu") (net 15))
 (segment (start 53.3069 77.9002) (end 54.9767 79.57) (width 0.2) (layer "B.Cu") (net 15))
 (segment (start 57.5639 79.0208) (end 59.0208 79.0208) (width 0.2) (layer "B.Cu") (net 15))
 (segment (start 28.3756 77.9002) (end 53.3069 77.9002) (width 0.2) (layer "B.Cu") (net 15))
 (segment (start 56.4438 80.9916) (end 57 80.4354) (width 0.2) (layer "B.Cu") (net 15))
 (segment (start 57 79.5847) (end 57.5639 79.0208) (width 0.2) (layer "B.Cu") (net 15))
 (segment (start 59.0208 79.0208) (end 60 80) (width 0.2) (layer "B.Cu") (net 15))
 (segment (start 16.11 60.97) (end 14.5216 62.5584) (width 0.2) (layer "B.Cu") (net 15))
 (segment (start 14.5216 62.5584) (end 14.5216 66.1345) (width 0.2) (layer "B.Cu") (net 15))
 (segment (start 62 41) (end 62 52) (width 0.2) (layer "F.Cu") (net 7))
 (segment (start 62 52) (end 62 63) (width 0.2) (layer "F.Cu") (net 7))
 (segment (start 62 30) (end 62 41) (width 0.2) (layer "F.Cu") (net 7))
 (segment (start 62 30) (end 60.3 31.7) (width 0.2) (layer "B.Cu") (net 7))
 (segment (start 17.44 31.7) (end 16.11 33.03) (width 0.2) (layer "B.Cu") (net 7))
 (segment (start 60.3 31.7) (end 17.44 31.7) (width 0.2) (layer "B.Cu") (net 7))
 (segment (start 63 80.4066) (end 63 79.543) (width 0.2) (layer "B.Cu") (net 14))
 (segment (start 58.995 80.995) (end 62.4116 80.995) (width 0.2) (layer "B.Cu") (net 14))
 (segment (start 22.46 64.78) (end 16.11 58.43) (width 0.2) (layer "B.Cu") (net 14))
 (segment (start 63 79.543) (end 48.237 64.78) (width 0.2) (layer "B.Cu") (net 14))
 (segment (start 48.237 64.78) (end 22.46 64.78) (width 0.2) (layer "B.Cu") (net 14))
 (segment (start 58 80) (end 58.995 80.995) (width 0.2) (layer "B.Cu") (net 14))
 (segment (start 62.4116 80.995) (end 63 80.4066) (width 0.2) (layer "B.Cu") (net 14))
 (segment (start 16.11 22.87) (end 16.11 24.0217) (width 0.2) (layer "F.Cu") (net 4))
 (segment (start 15.822 24.0217) (end 14.5146 25.3291) (width 0.2) (layer "F.Cu") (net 4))
 (segment (start 16.11 24.0217) (end 15.822 24.0217) (width 0.2) (layer "F.Cu") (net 4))
 (segment (start 14.5146 81.5146) (end 18 85) (width 0.2) (layer "F.Cu") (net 4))
 (segment (start 14.5146 25.3291) (end 14.5146 81.5146) (width 0.2) (layer "F.Cu") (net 4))
 (segment (start 20 29.3) (end 16.11 25.41) (width 0.2) (layer "F.Cu") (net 5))
 (segment (start 20 85) (end 20 29.3) (width 0.2) (layer "F.Cu") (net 5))
 (segment (start 52 80) (end 52 51.14) (width 0.2) (layer "F.Cu") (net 18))
 (segment (start 52 51.14) (end 33.89 33.03) (width 0.2) (layer "F.Cu") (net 18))
 (segment (start 52 80) (end 19.6104 80) (width 0.2) (layer "B.Cu") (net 18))
 (segment (start 19.6104 80) (end 14.9767 84.6337) (width 0.2) (layer "B.Cu") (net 18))
 (segment (start 14.9767 84.6337) (end 14.9767 85) (width 0.2) (layer "B.Cu") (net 18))
 (segment (start 14 85) (end 14.9767 85) (width 0.2) (layer "B.Cu") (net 18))
 (segment (start 60 30) (end 60 41) (width 0.2) (layer "F.Cu") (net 6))
 (segment (start 60 52) (end 60 41) (width 0.2) (layer "F.Cu") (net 6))
 (segment (start 60 63) (end 60 52) (width 0.2) (layer "F.Cu") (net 6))
 (segment (start 60 30) (end 59.0219 29.0219) (width 0.2) (layer "B.Cu") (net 6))
 (segment (start 43.6751 29.22) (end 17.38 29.22) (width 0.2) (layer "B.Cu") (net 6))
 (segment (start 43.8732 29.0219) (end 43.6751 29.22) (width 0.2) (layer "B.Cu") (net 6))
 (segment (start 59.0219 29.0219) (end 43.8732 29.0219) (width 0.2) (layer "B.Cu") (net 6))
 (segment (start 17.38 29.22) (end 16.11 30.49) (width 0.2) (layer "B.Cu") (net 6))
 (segment (start 14.9578 57.0422) (end 16.11 55.89) (width 0.2) (layer "B.Cu") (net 13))
 (segment (start 15.6732 64.78) (end 14.9416 64.0484) (width 0.2) (layer "B.Cu") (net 13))
 (segment (start 14.9416 64.0484) (end 14.9416 62.9836) (width 0.2) (layer "B.Cu") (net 13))
 (segment (start 14.9416 62.9836) (end 15.6852 62.24) (width 0.2) (layer "B.Cu") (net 13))
 (segment (start 56 80) (end 48.2817 72.2817) (width 0.2) (layer "B.Cu") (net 13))
 (segment (start 16.4719 59.7) (end 15.7175 59.7) (width 0.2) (layer "B.Cu") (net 13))
 (segment (start 24.1421 72.2817) (end 16.6404 64.78) (width 0.2) (layer "B.Cu") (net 13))
 (segment (start 15.6852 62.24) (end 16.4727 62.24) (width 0.2) (layer "B.Cu") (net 13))
 (segment (start 17.2617 61.451) (end 17.2617 60.4898) (width 0.2) (layer "B.Cu") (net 13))
 (segment (start 15.7175 59.7) (end 14.9578 58.9403) (width 0.2) (layer "B.Cu") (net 13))
 (segment (start 16.4727 62.24) (end 17.2617 61.451) (width 0.2) (layer "B.Cu") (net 13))
 (segment (start 14.9578 58.9403) (end 14.9578 57.0422) (width 0.2) (layer "B.Cu") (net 13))
 (segment (start 48.2817 72.2817) (end 24.1421 72.2817) (width 0.2) (layer "B.Cu") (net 13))
 (segment (start 16.6404 64.78) (end 15.6732 64.78) (width 0.2) (layer "B.Cu") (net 13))
 (segment (start 17.2617 60.4898) (end 16.4719 59.7) (width 0.2) (layer "B.Cu") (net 13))
 (segment (start 65.4733 18) (end 66.2 18) (width 0.2) (layer "F.Cu") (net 3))
 (segment (start 54 63) (end 54 52) (width 0.2) (layer "F.Cu") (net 3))
 (segment (start 65.4733 18) (end 65.4733 22) (width 0.2) (layer "F.Cu") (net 3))
 (segment (start 54.9767 29.6337) (end 54.9767 30) (width 0.2) (layer "F.Cu") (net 3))
 (segment (start 65.4733 18) (end 61.6 18) (width 0.2) (layer "F.Cu") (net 3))
 (segment (start 62.6104 22) (end 54.9767 29.6337) (width 0.2) (layer "F.Cu") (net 3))
 (segment (start 54 30) (end 54.9767 30) (width 0.2) (layer "F.Cu") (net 3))
 (segment (start 65.4733 22) (end 62.6104 22) (width 0.2) (layer "F.Cu") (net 3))
 (segment (start 54 41) (end 54 30) (width 0.2) (layer "F.Cu") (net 3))
 (segment (start 66.2 22) (end 65.4733 22) (width 0.2) (layer "F.Cu") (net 3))
 (segment (start 54 52) (end 54 41) (width 0.2) (layer "F.Cu") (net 3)))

